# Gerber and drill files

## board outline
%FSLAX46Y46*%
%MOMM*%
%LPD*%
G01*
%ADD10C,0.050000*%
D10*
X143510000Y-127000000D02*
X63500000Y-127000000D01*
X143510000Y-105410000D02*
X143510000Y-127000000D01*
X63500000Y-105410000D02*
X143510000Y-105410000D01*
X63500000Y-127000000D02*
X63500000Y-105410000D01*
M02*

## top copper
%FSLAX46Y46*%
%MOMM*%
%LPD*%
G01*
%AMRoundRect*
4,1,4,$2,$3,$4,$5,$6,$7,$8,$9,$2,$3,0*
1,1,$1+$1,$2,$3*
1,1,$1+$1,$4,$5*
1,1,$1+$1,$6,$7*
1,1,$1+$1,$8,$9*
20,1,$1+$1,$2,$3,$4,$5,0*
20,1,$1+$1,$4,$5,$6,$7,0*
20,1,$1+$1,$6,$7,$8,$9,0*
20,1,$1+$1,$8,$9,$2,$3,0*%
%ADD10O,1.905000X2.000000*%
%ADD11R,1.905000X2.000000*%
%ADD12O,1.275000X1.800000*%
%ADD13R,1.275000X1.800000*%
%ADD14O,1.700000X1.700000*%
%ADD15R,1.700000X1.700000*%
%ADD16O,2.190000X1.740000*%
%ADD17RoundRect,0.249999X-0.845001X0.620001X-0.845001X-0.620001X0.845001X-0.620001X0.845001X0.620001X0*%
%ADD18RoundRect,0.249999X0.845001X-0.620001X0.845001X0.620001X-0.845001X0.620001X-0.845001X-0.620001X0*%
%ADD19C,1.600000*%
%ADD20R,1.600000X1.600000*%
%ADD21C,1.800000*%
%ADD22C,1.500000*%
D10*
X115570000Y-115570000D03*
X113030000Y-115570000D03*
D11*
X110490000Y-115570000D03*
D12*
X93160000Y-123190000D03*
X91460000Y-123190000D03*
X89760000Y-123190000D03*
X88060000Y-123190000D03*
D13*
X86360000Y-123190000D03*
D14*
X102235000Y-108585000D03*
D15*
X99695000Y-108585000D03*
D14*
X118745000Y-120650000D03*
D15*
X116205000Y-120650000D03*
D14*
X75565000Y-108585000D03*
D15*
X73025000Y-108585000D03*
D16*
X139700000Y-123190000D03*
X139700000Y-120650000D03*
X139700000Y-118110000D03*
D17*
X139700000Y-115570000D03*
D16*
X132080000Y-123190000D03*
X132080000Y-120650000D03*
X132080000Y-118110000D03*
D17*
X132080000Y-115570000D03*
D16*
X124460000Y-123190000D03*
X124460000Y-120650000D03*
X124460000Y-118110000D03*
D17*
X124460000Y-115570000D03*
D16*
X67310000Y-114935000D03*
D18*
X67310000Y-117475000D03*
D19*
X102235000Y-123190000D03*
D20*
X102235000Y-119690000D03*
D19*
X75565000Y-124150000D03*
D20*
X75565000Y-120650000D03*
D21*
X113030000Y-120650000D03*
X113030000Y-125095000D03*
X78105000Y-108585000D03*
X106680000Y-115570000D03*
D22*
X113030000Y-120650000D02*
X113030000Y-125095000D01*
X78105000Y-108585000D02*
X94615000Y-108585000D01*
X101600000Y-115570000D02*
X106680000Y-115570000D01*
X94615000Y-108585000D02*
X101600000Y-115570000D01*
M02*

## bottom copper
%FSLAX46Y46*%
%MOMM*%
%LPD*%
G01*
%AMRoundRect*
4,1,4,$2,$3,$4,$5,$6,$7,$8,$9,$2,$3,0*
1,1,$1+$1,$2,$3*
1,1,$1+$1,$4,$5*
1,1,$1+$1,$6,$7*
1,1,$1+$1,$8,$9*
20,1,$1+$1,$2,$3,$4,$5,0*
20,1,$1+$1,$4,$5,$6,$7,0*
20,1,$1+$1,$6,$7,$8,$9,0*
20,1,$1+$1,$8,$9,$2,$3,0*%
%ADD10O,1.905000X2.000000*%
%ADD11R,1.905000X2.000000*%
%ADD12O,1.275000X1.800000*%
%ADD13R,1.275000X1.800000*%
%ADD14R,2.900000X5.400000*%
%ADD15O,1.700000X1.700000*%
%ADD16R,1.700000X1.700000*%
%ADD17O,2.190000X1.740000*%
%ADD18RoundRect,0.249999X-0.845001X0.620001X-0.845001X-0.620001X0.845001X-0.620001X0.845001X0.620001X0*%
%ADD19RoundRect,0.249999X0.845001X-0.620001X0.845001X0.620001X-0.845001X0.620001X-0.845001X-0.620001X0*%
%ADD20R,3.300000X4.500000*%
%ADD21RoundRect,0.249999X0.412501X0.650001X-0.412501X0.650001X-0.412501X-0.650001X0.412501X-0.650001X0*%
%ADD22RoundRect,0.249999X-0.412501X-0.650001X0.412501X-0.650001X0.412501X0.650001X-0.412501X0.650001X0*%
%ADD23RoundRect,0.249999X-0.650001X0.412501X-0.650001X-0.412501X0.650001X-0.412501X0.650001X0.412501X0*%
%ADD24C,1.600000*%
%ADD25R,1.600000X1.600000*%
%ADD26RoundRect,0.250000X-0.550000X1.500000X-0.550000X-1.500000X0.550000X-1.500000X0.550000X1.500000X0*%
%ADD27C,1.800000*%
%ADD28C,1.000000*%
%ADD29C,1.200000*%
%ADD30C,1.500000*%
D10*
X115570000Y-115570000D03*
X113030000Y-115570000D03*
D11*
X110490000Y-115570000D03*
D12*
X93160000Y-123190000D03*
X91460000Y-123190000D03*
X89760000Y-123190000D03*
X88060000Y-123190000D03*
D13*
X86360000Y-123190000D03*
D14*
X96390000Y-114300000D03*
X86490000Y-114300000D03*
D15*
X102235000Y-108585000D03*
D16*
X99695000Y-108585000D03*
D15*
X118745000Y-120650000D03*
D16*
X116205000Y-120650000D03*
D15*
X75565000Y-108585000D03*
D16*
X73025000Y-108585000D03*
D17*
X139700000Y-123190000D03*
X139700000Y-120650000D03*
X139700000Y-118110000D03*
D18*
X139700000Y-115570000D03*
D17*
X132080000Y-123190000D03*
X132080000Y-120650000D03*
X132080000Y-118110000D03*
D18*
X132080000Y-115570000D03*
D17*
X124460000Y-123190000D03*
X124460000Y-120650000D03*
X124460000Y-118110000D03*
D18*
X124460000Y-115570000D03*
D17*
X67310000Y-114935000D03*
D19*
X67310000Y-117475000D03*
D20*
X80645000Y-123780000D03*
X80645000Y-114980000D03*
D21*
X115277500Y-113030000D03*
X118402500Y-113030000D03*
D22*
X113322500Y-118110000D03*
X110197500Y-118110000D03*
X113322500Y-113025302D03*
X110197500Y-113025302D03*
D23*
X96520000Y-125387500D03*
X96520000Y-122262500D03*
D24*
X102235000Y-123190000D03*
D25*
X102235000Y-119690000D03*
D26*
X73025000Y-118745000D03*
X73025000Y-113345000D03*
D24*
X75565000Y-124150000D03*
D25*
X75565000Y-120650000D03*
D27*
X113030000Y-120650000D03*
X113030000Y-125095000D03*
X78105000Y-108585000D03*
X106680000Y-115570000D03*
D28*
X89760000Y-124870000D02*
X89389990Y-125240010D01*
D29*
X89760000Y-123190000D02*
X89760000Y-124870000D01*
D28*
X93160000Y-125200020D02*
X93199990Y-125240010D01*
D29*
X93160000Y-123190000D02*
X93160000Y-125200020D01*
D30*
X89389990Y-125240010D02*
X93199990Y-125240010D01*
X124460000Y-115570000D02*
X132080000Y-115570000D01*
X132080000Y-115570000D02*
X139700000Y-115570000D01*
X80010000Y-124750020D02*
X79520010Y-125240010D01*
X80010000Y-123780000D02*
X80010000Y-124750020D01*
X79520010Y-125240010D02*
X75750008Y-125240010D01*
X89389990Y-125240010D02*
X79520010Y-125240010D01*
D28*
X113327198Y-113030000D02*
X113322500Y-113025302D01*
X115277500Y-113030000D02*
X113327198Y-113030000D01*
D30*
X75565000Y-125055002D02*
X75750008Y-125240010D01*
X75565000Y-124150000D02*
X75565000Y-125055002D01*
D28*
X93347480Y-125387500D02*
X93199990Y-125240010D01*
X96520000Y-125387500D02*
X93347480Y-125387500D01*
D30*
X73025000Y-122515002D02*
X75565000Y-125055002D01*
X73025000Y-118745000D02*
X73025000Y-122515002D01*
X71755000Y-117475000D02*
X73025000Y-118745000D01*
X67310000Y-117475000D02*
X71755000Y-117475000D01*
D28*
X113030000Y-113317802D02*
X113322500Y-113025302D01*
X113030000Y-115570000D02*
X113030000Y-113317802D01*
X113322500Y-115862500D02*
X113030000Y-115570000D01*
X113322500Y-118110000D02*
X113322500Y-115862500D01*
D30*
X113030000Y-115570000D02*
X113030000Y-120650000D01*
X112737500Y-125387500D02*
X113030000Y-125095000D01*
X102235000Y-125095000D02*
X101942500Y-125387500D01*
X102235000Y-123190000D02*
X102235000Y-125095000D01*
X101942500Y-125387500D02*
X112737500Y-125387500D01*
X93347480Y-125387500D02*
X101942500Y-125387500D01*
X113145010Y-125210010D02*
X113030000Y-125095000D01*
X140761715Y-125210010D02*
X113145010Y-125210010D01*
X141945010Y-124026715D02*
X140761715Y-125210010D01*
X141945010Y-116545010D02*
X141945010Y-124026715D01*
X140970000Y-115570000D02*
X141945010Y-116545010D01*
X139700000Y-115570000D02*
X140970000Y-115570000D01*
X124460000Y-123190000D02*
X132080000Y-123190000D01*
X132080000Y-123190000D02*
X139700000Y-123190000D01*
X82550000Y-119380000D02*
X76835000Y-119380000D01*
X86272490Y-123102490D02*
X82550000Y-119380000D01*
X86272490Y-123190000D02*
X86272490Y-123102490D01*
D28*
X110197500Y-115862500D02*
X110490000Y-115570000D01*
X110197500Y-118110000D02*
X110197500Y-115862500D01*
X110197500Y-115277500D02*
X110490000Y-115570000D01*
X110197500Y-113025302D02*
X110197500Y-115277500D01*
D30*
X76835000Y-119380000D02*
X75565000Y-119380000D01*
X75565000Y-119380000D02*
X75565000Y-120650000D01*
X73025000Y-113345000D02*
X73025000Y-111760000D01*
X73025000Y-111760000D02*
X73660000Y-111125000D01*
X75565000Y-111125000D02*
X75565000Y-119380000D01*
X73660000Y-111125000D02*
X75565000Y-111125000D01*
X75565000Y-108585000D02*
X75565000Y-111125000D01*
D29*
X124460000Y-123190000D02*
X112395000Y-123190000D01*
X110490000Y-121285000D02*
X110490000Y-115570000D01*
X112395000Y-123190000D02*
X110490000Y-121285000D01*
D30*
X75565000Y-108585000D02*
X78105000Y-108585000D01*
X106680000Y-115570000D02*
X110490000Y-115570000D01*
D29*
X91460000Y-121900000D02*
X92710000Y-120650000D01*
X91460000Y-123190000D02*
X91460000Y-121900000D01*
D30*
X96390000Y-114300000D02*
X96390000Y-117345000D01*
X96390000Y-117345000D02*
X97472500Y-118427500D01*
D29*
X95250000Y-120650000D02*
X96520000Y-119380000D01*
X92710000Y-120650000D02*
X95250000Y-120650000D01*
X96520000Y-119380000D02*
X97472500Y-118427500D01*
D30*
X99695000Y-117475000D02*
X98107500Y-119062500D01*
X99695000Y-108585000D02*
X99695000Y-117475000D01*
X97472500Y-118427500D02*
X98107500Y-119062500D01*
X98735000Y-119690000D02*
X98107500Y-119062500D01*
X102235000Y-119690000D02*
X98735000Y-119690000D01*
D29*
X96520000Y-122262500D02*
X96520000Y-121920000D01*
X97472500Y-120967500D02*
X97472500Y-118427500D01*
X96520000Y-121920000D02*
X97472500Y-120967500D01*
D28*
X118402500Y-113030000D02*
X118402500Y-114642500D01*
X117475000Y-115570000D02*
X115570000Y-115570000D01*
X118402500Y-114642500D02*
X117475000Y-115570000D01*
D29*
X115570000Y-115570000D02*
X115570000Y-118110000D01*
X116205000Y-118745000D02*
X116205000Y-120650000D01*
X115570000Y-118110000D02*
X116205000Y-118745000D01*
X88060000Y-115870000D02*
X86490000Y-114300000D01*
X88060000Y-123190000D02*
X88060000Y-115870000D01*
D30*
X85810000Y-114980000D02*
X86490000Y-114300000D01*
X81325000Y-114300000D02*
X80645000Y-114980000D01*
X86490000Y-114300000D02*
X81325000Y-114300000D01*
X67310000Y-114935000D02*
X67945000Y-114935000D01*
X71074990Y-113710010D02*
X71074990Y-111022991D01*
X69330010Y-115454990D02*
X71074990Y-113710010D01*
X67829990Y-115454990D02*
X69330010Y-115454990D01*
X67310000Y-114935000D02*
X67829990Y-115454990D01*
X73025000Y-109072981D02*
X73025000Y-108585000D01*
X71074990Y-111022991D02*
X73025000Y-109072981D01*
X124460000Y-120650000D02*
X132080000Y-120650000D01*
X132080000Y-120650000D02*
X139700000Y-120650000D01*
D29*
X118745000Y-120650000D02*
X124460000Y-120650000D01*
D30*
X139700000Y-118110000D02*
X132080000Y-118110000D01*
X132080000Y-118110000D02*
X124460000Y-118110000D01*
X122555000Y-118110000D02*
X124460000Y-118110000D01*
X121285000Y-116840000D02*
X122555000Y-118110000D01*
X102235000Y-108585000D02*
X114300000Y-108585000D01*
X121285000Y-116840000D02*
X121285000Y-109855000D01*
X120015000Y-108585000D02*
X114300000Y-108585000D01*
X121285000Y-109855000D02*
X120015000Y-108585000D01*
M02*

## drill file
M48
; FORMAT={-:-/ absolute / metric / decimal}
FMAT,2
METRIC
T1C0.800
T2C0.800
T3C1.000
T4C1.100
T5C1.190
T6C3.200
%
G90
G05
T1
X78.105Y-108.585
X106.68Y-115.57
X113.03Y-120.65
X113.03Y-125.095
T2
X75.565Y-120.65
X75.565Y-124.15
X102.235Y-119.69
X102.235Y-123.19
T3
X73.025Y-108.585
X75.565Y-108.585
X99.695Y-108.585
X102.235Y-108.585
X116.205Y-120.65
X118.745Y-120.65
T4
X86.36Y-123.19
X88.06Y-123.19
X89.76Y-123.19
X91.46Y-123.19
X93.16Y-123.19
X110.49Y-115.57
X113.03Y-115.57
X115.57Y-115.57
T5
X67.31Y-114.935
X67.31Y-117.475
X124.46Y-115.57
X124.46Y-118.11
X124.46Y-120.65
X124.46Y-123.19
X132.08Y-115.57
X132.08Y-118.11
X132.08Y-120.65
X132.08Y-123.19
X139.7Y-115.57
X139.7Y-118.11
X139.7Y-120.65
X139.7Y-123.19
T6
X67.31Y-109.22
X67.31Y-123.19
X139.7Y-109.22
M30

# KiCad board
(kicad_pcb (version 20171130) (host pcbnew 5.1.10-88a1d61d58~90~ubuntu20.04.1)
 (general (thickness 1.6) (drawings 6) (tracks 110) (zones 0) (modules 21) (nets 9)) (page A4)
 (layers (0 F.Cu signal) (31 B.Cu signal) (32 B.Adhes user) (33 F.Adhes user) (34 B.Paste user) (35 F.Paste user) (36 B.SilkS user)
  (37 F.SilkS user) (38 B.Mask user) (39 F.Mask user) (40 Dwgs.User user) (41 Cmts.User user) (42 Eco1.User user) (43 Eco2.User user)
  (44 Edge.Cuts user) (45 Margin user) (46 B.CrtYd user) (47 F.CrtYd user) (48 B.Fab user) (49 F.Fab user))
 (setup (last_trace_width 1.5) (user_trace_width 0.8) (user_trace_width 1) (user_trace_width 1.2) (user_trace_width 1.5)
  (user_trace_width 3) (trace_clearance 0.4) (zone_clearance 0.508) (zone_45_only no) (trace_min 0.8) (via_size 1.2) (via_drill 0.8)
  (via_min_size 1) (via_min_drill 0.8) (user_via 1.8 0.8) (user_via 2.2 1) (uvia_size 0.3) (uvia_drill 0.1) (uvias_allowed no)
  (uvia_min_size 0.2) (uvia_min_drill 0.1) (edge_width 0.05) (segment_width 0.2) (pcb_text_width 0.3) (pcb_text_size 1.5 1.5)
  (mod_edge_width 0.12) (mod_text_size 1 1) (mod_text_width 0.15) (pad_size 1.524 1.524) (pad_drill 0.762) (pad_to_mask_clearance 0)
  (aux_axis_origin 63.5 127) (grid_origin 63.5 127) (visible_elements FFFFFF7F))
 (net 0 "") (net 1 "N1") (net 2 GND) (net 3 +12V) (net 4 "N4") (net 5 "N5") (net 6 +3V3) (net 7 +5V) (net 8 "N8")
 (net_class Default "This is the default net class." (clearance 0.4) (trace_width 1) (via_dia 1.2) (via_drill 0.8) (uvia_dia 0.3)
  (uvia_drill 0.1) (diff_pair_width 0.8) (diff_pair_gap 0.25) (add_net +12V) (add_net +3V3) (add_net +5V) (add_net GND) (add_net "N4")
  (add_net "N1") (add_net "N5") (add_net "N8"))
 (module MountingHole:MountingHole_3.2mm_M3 (layer F.Cu) (at 139.7 109.22)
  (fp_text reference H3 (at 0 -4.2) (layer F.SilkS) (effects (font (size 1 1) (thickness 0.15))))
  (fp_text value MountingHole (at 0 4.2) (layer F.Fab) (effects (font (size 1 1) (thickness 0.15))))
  (pad 1 np_thru_hole circle (at 0 0) (size 3.2 3.2) (drill 3.2) (layers *.Cu *.Mask)))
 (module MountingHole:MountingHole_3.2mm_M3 (layer F.Cu) (at 67.31 123.19)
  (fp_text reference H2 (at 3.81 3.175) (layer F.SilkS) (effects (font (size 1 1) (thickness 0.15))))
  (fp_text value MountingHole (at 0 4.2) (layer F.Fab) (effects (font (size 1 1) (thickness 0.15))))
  (pad 1 np_thru_hole circle (at 0 0) (size 3.2 3.2) (drill 3.2) (layers *.Cu *.Mask)))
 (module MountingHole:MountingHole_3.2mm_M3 (layer F.Cu) (at 67.31 109.22)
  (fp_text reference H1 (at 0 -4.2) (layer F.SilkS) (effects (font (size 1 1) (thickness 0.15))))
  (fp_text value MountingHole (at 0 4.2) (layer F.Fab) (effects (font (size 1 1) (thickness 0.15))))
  (pad 1 np_thru_hole circle (at 0 0) (size 3.2 3.2) (drill 3.2) (layers *.Cu *.Mask)))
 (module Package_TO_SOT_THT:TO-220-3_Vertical (layer F.Cu) (at 110.49 115.57)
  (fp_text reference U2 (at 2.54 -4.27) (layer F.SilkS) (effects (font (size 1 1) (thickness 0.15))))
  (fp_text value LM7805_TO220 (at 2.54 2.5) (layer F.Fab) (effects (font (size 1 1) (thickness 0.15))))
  (pad 3 thru_hole oval (at 5.08 0) (size 1.905 2) (drill 1.1) (layers *.Cu *.Mask) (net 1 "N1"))
  (pad 2 thru_hole oval (at 2.54 0) (size 1.905 2) (drill 1.1) (layers *.Cu *.Mask) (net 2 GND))
  (pad 1 thru_hole rect (at 0 0) (size 1.905 2) (drill 1.1) (layers *.Cu *.Mask) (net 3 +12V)))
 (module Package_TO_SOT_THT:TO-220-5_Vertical (layer F.Cu) (at 86.36 123.19)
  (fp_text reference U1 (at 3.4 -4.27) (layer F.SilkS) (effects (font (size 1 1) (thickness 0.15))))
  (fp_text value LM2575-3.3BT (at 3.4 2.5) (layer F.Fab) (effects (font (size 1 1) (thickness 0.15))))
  (pad 5 thru_hole oval (at 6.8 0) (size 1.275 1.8) (drill 1.1) (layers *.Cu *.Mask) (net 2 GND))
  (pad 4 thru_hole oval (at 5.1 0) (size 1.275 1.8) (drill 1.1) (layers *.Cu *.Mask) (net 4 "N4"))
  (pad 3 thru_hole oval (at 3.4 0) (size 1.275 1.8) (drill 1.1) (layers *.Cu *.Mask) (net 2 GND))
  (pad 2 thru_hole oval (at 1.7 0) (size 1.275 1.8) (drill 1.1) (layers *.Cu *.Mask) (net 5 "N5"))
  (pad 1 thru_hole rect (at 0 0) (size 1.275 1.8) (drill 1.1) (layers *.Cu *.Mask) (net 3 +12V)))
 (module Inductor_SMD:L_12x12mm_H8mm (layer B.Cu) (at 91.44 114.3)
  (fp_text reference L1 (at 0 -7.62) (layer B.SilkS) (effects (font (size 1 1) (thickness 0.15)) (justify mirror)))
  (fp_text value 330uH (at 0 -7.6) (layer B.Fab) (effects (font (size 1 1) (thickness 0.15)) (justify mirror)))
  (pad 2 smd rect (at 4.95 0) (size 2.9 5.4) (layers B.Cu B.Paste B.Mask) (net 4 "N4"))
  (pad 1 smd rect (at -4.95 0) (size 2.9 5.4) (layers B.Cu B.Paste B.Mask) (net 5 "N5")))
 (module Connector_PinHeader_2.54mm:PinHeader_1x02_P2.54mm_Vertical (layer F.Cu) (at 99.695 108.585 90)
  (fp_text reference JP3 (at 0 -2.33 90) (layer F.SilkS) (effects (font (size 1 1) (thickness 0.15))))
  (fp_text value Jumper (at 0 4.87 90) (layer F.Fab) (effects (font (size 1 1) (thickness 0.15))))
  (pad 2 thru_hole oval (at 0 2.54 90) (size 1.7 1.7) (drill 1) (layers *.Cu *.Mask) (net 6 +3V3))
  (pad 1 thru_hole rect (at 0 0 90) (size 1.7 1.7) (drill 1) (layers *.Cu *.Mask) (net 4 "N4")))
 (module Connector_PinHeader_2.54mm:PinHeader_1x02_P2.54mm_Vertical (layer F.Cu) (at 116.205 120.65 90)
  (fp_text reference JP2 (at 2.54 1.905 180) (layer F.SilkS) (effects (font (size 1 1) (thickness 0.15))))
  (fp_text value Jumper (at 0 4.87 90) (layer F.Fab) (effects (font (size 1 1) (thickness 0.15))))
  (pad 2 thru_hole oval (at 0 2.54 90) (size 1.7 1.7) (drill 1) (layers *.Cu *.Mask) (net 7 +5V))
  (pad 1 thru_hole rect (at 0 0 90) (size 1.7 1.7) (drill 1) (layers *.Cu *.Mask) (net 1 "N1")))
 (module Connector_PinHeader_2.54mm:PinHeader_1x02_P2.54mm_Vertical (layer F.Cu) (at 73.025 108.585 90)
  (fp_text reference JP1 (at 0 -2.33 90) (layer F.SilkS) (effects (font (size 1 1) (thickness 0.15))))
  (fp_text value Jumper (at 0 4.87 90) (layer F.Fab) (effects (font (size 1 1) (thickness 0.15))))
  (pad 2 thru_hole oval (at 0 2.54 90) (size 1.7 1.7) (drill 1) (layers *.Cu *.Mask) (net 3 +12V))
  (pad 1 thru_hole rect (at 0 0 90) (size 1.7 1.7) (drill 1) (layers *.Cu *.Mask) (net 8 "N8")))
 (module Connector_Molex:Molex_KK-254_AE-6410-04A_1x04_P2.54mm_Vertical (layer F.Cu) (at 139.7 115.57 270)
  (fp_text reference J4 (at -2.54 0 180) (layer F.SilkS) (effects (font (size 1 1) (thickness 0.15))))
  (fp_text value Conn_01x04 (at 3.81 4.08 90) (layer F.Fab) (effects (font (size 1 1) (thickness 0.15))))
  (pad 4 thru_hole oval (at 7.62 0 270) (size 1.74 2.19) (drill 1.19) (layers *.Cu *.Mask) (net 3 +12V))
  (pad 3 thru_hole oval (at 5.08 0 270) (size 1.74 2.19) (drill 1.19) (layers *.Cu *.Mask) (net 7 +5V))
  (pad 2 thru_hole oval (at 2.54 0 270) (size 1.74 2.19) (drill 1.19) (layers *.Cu *.Mask) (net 6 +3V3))
  (pad 1 thru_hole roundrect (at 0 0 270) (size 1.74 2.19) (drill 1.19) (layers *.Cu *.Mask) (roundrect_rratio 0.1436775862068966)
   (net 2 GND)))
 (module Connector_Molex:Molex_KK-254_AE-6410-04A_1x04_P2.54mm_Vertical (layer F.Cu) (at 132.08 115.57 270)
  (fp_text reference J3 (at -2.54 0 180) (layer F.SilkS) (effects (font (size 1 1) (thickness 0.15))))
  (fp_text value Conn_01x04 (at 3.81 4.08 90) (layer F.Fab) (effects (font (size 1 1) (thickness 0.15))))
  (pad 4 thru_hole oval (at 7.62 0 270) (size 1.74 2.19) (drill 1.19) (layers *.Cu *.Mask) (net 3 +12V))
  (pad 3 thru_hole oval (at 5.08 0 270) (size 1.74 2.19) (drill 1.19) (layers *.Cu *.Mask) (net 7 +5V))
  (pad 2 thru_hole oval (at 2.54 0 270) (size 1.74 2.19) (drill 1.19) (layers *.Cu *.Mask) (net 6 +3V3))
  (pad 1 thru_hole roundrect (at 0 0 270) (size 1.74 2.19) (drill 1.19) (layers *.Cu *.Mask) (roundrect_rratio 0.1436775862068966)
   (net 2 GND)))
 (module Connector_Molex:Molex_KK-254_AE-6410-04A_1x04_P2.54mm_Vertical (layer F.Cu) (at 124.46 115.57 270)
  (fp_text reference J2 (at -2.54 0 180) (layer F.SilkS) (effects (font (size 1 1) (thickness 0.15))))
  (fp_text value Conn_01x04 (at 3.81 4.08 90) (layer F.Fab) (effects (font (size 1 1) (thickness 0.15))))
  (pad 4 thru_hole oval (at 7.62 0 270) (size 1.74 2.19) (drill 1.19) (layers *.Cu *.Mask) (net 3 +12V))
  (pad 3 thru_hole oval (at 5.08 0 270) (size 1.74 2.19) (drill 1.19) (layers *.Cu *.Mask) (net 7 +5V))
  (pad 2 thru_hole oval (at 2.54 0 270) (size 1.74 2.19) (drill 1.19) (layers *.Cu *.Mask) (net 6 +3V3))
  (pad 1 thru_hole roundrect (at 0 0 270) (size 1.74 2.19) (drill 1.19) (layers *.Cu *.Mask) (roundrect_rratio 0.1436775862068966)
   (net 2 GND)))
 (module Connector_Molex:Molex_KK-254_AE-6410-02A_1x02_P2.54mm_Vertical (layer F.Cu) (at 67.31 117.475 90)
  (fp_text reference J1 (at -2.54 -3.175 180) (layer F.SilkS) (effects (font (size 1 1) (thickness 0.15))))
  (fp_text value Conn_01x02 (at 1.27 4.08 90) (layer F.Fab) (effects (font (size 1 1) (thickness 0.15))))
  (pad 2 thru_hole oval (at 2.54 0 90) (size 1.74 2.19) (drill 1.19) (layers *.Cu *.Mask) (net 8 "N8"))
  (pad 1 thru_hole roundrect (at 0 0 90) (size 1.74 2.19) (drill 1.19) (layers *.Cu *.Mask) (roundrect_rratio 0.1436775862068966)
   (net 2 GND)))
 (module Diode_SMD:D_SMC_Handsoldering (layer B.Cu) (at 80.645 119.38 270)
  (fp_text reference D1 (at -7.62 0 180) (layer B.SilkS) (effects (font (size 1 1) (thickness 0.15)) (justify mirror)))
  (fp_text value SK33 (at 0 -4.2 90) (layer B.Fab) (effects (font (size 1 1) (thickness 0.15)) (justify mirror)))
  (pad 2 smd rect (at 4.4 0 180) (size 3.3 4.5) (layers B.Cu B.Paste B.Mask) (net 2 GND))
  (pad 1 smd rect (at -4.4 0 180) (size 3.3 4.5) (layers B.Cu B.Paste B.Mask) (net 5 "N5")))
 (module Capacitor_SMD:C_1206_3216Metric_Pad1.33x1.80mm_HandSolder (layer B.Cu) (at 116.84 113.03 180)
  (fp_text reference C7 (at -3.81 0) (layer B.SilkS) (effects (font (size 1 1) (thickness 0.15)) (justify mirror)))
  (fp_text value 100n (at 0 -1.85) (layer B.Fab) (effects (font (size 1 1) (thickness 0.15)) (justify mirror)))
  (pad 2 smd roundrect (at 1.5625 0 180) (size 1.325 1.8) (layers B.Cu B.Paste B.Mask) (roundrect_rratio 0.1886784905660377) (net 2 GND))
  (pad 1 smd roundrect (at -1.5625 0 180) (size 1.325 1.8) (layers B.Cu B.Paste B.Mask) (roundrect_rratio 0.1886784905660377) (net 1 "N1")))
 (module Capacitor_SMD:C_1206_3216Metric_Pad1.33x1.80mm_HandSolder (layer B.Cu) (at 111.76 118.11)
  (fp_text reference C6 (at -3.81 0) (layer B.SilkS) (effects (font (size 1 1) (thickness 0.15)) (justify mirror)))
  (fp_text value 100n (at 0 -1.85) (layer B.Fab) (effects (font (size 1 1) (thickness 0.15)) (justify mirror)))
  (pad 2 smd roundrect (at 1.5625 0) (size 1.325 1.8) (layers B.Cu B.Paste B.Mask) (roundrect_rratio 0.1886784905660377) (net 2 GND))
  (pad 1 smd roundrect (at -1.5625 0) (size 1.325 1.8) (layers B.Cu B.Paste B.Mask) (roundrect_rratio 0.1886784905660377) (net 3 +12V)))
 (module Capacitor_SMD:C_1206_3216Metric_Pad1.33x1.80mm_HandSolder (layer B.Cu) (at 111.76 113.025302)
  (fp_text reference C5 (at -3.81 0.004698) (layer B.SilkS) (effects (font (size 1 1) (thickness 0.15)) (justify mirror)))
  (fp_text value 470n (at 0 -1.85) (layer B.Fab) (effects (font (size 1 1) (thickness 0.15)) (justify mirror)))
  (pad 2 smd roundrect (at 1.5625 0) (size 1.325 1.8) (layers B.Cu B.Paste B.Mask) (roundrect_rratio 0.1886784905660377) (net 2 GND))
  (pad 1 smd roundrect (at -1.5625 0) (size 1.325 1.8) (layers B.Cu B.Paste B.Mask) (roundrect_rratio 0.1886784905660377) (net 3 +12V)))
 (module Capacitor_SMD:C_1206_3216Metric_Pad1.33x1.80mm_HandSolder (layer B.Cu) (at 96.52 123.825 270)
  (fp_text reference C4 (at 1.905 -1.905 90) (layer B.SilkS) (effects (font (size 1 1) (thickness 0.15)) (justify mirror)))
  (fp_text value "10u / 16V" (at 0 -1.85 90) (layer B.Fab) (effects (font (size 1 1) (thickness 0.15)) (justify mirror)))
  (pad 2 smd roundrect (at 1.5625 0 270) (size 1.325 1.8) (layers B.Cu B.Paste B.Mask) (roundrect_rratio 0.1886784905660377) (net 2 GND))
  (pad 1 smd roundrect (at -1.5625 0 270) (size 1.325 1.8) (layers B.Cu B.Paste B.Mask) (roundrect_rratio 0.1886784905660377) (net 4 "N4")))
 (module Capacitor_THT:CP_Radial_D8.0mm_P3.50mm (layer F.Cu) (at 102.235 119.69 270)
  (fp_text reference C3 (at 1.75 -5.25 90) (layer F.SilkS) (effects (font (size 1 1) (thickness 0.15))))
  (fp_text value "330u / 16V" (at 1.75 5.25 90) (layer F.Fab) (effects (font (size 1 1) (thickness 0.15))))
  (pad 2 thru_hole circle (at 3.5 0 270) (size 1.6 1.6) (drill 0.8) (layers *.Cu *.Mask) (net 2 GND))
  (pad 1 thru_hole rect (at 0 0 270) (size 1.6 1.6) (drill 0.8) (layers *.Cu *.Mask) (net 4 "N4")))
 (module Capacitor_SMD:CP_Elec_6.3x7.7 (layer B.Cu) (at 73.025 116.045 270)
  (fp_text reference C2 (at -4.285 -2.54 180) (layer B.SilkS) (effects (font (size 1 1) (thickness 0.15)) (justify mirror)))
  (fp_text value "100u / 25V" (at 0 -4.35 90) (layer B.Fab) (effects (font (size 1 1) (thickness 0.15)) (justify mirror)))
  (pad 2 smd roundrect (at 2.7 0 270) (size 3.5 1.6) (layers B.Cu B.Paste B.Mask) (roundrect_rratio 0.15625) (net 2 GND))
  (pad 1 smd roundrect (at -2.7 0 270) (size 3.5 1.6) (layers B.Cu B.Paste B.Mask) (roundrect_rratio 0.15625) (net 3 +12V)))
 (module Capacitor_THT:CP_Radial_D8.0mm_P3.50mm (layer F.Cu) (at 75.565 120.65 270)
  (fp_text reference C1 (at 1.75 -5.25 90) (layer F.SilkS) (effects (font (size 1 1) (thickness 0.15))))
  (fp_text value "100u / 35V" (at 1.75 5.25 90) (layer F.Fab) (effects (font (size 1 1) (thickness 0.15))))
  (pad 2 thru_hole circle (at 3.5 0 270) (size 1.6 1.6) (drill 0.8) (layers *.Cu *.Mask) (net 2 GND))
  (pad 1 thru_hole rect (at 0 0 270) (size 1.6 1.6) (drill 0.8) (layers *.Cu *.Mask) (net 3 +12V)))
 (gr_line (start 143.51 127) (end 63.5 127) (layer Edge.Cuts) (width 0.05))
 (gr_line (start 143.51 105.41) (end 143.51 127) (layer Edge.Cuts) (width 0.05))
 (gr_line (start 63.5 105.41) (end 143.51 105.41) (layer Edge.Cuts) (width 0.05))
 (gr_line (start 63.5 127) (end 63.5 105.41) (layer Edge.Cuts) (width 0.05))
 (segment (start 89.76 124.87) (end 89.38999 125.24001) (width 1) (layer B.Cu) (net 2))
 (segment (start 89.76 123.19) (end 89.76 124.87) (width 1.2) (layer B.Cu) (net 2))
 (segment (start 93.16 125.20002) (end 93.19999 125.24001) (width 1) (layer B.Cu) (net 2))
 (segment (start 93.16 123.19) (end 93.16 125.20002) (width 1.2) (layer B.Cu) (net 2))
 (segment (start 89.38999 125.24001) (end 93.19999 125.24001) (width 1.5) (layer B.Cu) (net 2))
 (segment (start 124.46 115.57) (end 132.08 115.57) (width 1.5) (layer B.Cu) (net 2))
 (segment (start 132.08 115.57) (end 139.7 115.57) (width 1.5) (layer B.Cu) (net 2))
 (segment (start 80.01 124.75002) (end 79.52001 125.24001) (width 1.5) (layer B.Cu) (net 2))
 (segment (start 80.01 123.78) (end 80.01 124.75002) (width 1.5) (layer B.Cu) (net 2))
 (segment (start 79.52001 125.24001) (end 75.750008 125.24001) (width 1.5) (layer B.Cu) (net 2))
 (segment (start 89.38999 125.24001) (end 79.52001 125.24001) (width 1.5) (layer B.Cu) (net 2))
 (segment (start 113.327198 113.03) (end 113.3225 113.025302) (width 1) (layer B.Cu) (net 2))
 (segment (start 115.2775 113.03) (end 113.327198 113.03) (width 1) (layer B.Cu) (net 2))
 (segment (start 75.565 125.055002) (end 75.750008 125.24001) (width 1.5) (layer B.Cu) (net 2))
 (segment (start 75.565 124.15) (end 75.565 125.055002) (width 1.5) (layer B.Cu) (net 2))
 (segment (start 93.34748 125.3875) (end 93.19999 125.24001) (width 1) (layer B.Cu) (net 2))
 (segment (start 96.52 125.3875) (end 93.34748 125.3875) (width 1) (layer B.Cu) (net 2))
 (segment (start 73.025 122.515002) (end 75.565 125.055002) (width 1.5) (layer B.Cu) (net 2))
 (segment (start 73.025 118.745) (end 73.025 122.515002) (width 1.5) (layer B.Cu) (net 2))
 (segment (start 71.755 117.475) (end 73.025 118.745) (width 1.5) (layer B.Cu) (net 2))
 (segment (start 67.31 117.475) (end 71.755 117.475) (width 1.5) (layer B.Cu) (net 2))
 (segment (start 113.03 113.317802) (end 113.3225 113.025302) (width 1) (layer B.Cu) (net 2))
 (segment (start 113.03 115.57) (end 113.03 113.317802) (width 1) (layer B.Cu) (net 2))
 (segment (start 113.3225 115.8625) (end 113.03 115.57) (width 1) (layer B.Cu) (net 2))
 (segment (start 113.3225 118.11) (end 113.3225 115.8625) (width 1) (layer B.Cu) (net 2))
 (via (at 113.03 120.65) (size 1.8) (drill 0.8) (layers F.Cu B.Cu) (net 2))
 (segment (start 113.03 115.57) (end 113.03 120.65) (width 1.5) (layer B.Cu) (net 2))
 (via (at 113.03 125.095) (size 1.8) (drill 0.8) (layers F.Cu B.Cu) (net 2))
 (segment (start 113.03 120.65) (end 113.03 125.095) (width 1.5) (layer F.Cu) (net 2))
 (segment (start 112.7375 125.3875) (end 113.03 125.095) (width 1.5) (layer B.Cu) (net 2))
 (segment (start 102.235 125.095) (end 101.9425 125.3875) (width 1.5) (layer B.Cu) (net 2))
 (segment (start 102.235 123.19) (end 102.235 125.095) (width 1.5) (layer B.Cu) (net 2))
 (segment (start 101.9425 125.3875) (end 112.7375 125.3875) (width 1.5) (layer B.Cu) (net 2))
 (segment (start 93.34748 125.3875) (end 101.9425 125.3875) (width 1.5) (layer B.Cu) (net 2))
 (segment (start 113.14501 125.21001) (end 113.03 125.095) (width 1.5) (layer B.Cu) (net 2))
 (segment (start 140.761715 125.21001) (end 113.14501 125.21001) (width 1.5) (layer B.Cu) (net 2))
 (segment (start 141.94501 124.026715) (end 140.761715 125.21001) (width 1.5) (layer B.Cu) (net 2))
 (segment (start 141.94501 116.54501) (end 141.94501 124.026715) (width 1.5) (layer B.Cu) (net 2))
 (segment (start 140.97 115.57) (end 141.94501 116.54501) (width 1.5) (layer B.Cu) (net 2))
 (segment (start 139.7 115.57) (end 140.97 115.57) (width 1.5) (layer B.Cu) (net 2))
 (segment (start 124.46 123.19) (end 132.08 123.19) (width 1.5) (layer B.Cu) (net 3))
 (segment (start 132.08 123.19) (end 139.7 123.19) (width 1.5) (layer B.Cu) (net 3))
 (segment (start 82.55 119.38) (end 76.835 119.38) (width 1.5) (layer B.Cu) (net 3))
 (segment (start 86.27249 123.10249) (end 82.55 119.38) (width 1.5) (layer B.Cu) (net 3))
 (segment (start 86.27249 123.19) (end 86.27249 123.10249) (width 1.5) (layer B.Cu) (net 3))
 (segment (start 110.1975 115.8625) (end 110.49 115.57) (width 1) (layer B.Cu) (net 3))
 (segment (start 110.1975 118.11) (end 110.1975 115.8625) (width 1) (layer B.Cu) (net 3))
 (segment (start 110.1975 115.2775) (end 110.49 115.57) (width 1) (layer B.Cu) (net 3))
 (segment (start 110.1975 113.025302) (end 110.1975 115.2775) (width 1) (layer B.Cu) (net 3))
 (segment (start 76.835 119.38) (end 75.565 119.38) (width 1.5) (layer B.Cu) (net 3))
 (segment (start 75.565 119.38) (end 75.565 120.65) (width 1.5) (layer B.Cu) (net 3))
 (segment (start 73.025 113.345) (end 73.025 111.76) (width 1.5) (layer B.Cu) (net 3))
 (segment (start 73.025 111.76) (end 73.66 111.125) (width 1.5) (layer B.Cu) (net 3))
 (segment (start 75.565 111.125) (end 75.565 119.38) (width 1.5) (layer B.Cu) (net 3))
 (segment (start 73.66 111.125) (end 75.565 111.125) (width 1.5) (layer B.Cu) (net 3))
 (segment (start 75.565 108.585) (end 75.565 111.125) (width 1.5) (layer B.Cu) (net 3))
 (segment (start 124.46 123.19) (end 112.395 123.19) (width 1.2) (layer B.Cu) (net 3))
 (segment (start 110.49 121.285) (end 110.49 115.57) (width 1.2) (layer B.Cu) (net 3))
 (segment (start 112.395 123.19) (end 110.49 121.285) (width 1.2) (layer B.Cu) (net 3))
 (via (at 78.105 108.585) (size 1.8) (drill 0.8) (layers F.Cu B.Cu) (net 3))
 (segment (start 75.565 108.585) (end 78.105 108.585) (width 1.5) (layer B.Cu) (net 3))
 (segment (start 78.105 108.585) (end 94.615 108.585) (width 1.5) (layer F.Cu) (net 3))
 (via (at 106.68 115.57) (size 1.8) (drill 0.8) (layers F.Cu B.Cu) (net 3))
 (segment (start 101.6 115.57) (end 106.68 115.57) (width 1.5) (layer F.Cu) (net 3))
 (segment (start 94.615 108.585) (end 101.6 115.57) (width 1.5) (layer F.Cu) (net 3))
 (segment (start 106.68 115.57) (end 110.49 115.57) (width 1.5) (layer B.Cu) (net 3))
 (segment (start 91.46 121.9) (end 92.71 120.65) (width 1.2) (layer B.Cu) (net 4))
 (segment (start 91.46 123.19) (end 91.46 121.9) (width 1.2) (layer B.Cu) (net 4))
 (segment (start 96.39 114.3) (end 96.39 117.345) (width 1.5) (layer B.Cu) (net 4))
 (segment (start 96.39 117.345) (end 97.4725 118.4275) (width 1.5) (layer B.Cu) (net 4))
 (segment (start 95.25 120.65) (end 96.52 119.38) (width 1.2) (layer B.Cu) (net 4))
 (segment (start 92.71 120.65) (end 95.25 120.65) (width 1.2) (layer B.Cu) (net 4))
 (segment (start 96.52 119.38) (end 97.4725 118.4275) (width 1.2) (layer B.Cu) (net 4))
 (segment (start 99.695 117.475) (end 98.1075 119.0625) (width 1.5) (layer B.Cu) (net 4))
 (segment (start 99.695 108.585) (end 99.695 117.475) (width 1.5) (layer B.Cu) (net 4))
 (segment (start 97.4725 118.4275) (end 98.1075 119.0625) (width 1.5) (layer B.Cu) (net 4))
 (segment (start 98.735 119.69) (end 98.1075 119.0625) (width 1.5) (layer B.Cu) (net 4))
 (segment (start 102.235 119.69) (end 98.735 119.69) (width 1.5) (layer B.Cu) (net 4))
 (segment (start 96.52 122.2625) (end 96.52 121.92) (width 1.2) (layer B.Cu) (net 4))
 (segment (start 97.4725 120.9675) (end 97.4725 118.4275) (width 1.2) (layer B.Cu) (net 4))
 (segment (start 96.52 121.92) (end 97.4725 120.9675) (width 1.2) (layer B.Cu) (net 4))
 (segment (start 118.4025 113.03) (end 118.4025 114.6425) (width 1) (layer B.Cu) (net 1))
 (segment (start 117.475 115.57) (end 115.57 115.57) (width 1) (layer B.Cu) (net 1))
 (segment (start 118.4025 114.6425) (end 117.475 115.57) (width 1) (layer B.Cu) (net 1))
 (segment (start 115.57 115.57) (end 115.57 118.11) (width 1.2) (layer B.Cu) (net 1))
 (segment (start 116.205 118.745) (end 116.205 120.65) (width 1.2) (layer B.Cu) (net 1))
 (segment (start 115.57 118.11) (end 116.205 118.745) (width 1.2) (layer B.Cu) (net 1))
 (segment (start 88.06 115.87) (end 86.49 114.3) (width 1.2) (layer B.Cu) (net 5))
 (segment (start 88.06 123.19) (end 88.06 115.87) (width 1.2) (layer B.Cu) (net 5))
 (segment (start 85.81 114.98) (end 86.49 114.3) (width 1.5) (layer B.Cu) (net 5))
 (segment (start 81.325 114.3) (end 80.645 114.98) (width 1.5) (layer B.Cu) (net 5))
 (segment (start 86.49 114.3) (end 81.325 114.3) (width 1.5) (layer B.Cu) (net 5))
 (segment (start 67.31 114.935) (end 67.945 114.935) (width 1.5) (layer B.Cu) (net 8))
 (segment (start 71.07499 113.71001) (end 71.07499 111.022991) (width 1.5) (layer B.Cu) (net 8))
 (segment (start 69.33001 115.45499) (end 71.07499 113.71001) (width 1.5) (layer B.Cu) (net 8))
 (segment (start 67.82999 115.45499) (end 69.33001 115.45499) (width 1.5) (layer B.Cu) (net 8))
 (segment (start 67.31 114.935) (end 67.82999 115.45499) (width 1.5) (layer B.Cu) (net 8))
 (segment (start 73.025 109.072981) (end 73.025 108.585) (width 1.5) (layer B.Cu) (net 8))
 (segment (start 71.07499 111.022991) (end 73.025 109.072981) (width 1.5) (layer B.Cu) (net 8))
 (segment (start 124.46 120.65) (end 132.08 120.65) (width 1.5) (layer B.Cu) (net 7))
 (segment (start 132.08 120.65) (end 139.7 120.65) (width 1.5) (layer B.Cu) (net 7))
 (segment (start 118.745 120.65) (end 124.46 120.65) (width 1.2) (layer B.Cu) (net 7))
 (segment (start 139.7 118.11) (end 132.08 118.11) (width 1.5) (layer B.Cu) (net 6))
 (segment (start 132.08 118.11) (end 124.46 118.11) (width 1.5) (layer B.Cu) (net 6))
 (segment (start 122.555 118.11) (end 124.46 118.11) (width 1.5) (layer B.Cu) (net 6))
 (segment (start 121.285 116.84) (end 122.555 118.11) (width 1.5) (layer B.Cu) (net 6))
 (segment (start 102.235 108.585) (end 114.3 108.585) (width 1.5) (layer B.Cu) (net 6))
 (segment (start 121.285 116.84) (end 121.285 109.855) (width 1.5) (layer B.Cu) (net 6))
 (segment (start 120.015 108.585) (end 114.3 108.585) (width 1.5) (layer B.Cu) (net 6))
 (segment (start 121.285 109.855) (end 120.015 108.585) (width 1.5) (layer B.Cu) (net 6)))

